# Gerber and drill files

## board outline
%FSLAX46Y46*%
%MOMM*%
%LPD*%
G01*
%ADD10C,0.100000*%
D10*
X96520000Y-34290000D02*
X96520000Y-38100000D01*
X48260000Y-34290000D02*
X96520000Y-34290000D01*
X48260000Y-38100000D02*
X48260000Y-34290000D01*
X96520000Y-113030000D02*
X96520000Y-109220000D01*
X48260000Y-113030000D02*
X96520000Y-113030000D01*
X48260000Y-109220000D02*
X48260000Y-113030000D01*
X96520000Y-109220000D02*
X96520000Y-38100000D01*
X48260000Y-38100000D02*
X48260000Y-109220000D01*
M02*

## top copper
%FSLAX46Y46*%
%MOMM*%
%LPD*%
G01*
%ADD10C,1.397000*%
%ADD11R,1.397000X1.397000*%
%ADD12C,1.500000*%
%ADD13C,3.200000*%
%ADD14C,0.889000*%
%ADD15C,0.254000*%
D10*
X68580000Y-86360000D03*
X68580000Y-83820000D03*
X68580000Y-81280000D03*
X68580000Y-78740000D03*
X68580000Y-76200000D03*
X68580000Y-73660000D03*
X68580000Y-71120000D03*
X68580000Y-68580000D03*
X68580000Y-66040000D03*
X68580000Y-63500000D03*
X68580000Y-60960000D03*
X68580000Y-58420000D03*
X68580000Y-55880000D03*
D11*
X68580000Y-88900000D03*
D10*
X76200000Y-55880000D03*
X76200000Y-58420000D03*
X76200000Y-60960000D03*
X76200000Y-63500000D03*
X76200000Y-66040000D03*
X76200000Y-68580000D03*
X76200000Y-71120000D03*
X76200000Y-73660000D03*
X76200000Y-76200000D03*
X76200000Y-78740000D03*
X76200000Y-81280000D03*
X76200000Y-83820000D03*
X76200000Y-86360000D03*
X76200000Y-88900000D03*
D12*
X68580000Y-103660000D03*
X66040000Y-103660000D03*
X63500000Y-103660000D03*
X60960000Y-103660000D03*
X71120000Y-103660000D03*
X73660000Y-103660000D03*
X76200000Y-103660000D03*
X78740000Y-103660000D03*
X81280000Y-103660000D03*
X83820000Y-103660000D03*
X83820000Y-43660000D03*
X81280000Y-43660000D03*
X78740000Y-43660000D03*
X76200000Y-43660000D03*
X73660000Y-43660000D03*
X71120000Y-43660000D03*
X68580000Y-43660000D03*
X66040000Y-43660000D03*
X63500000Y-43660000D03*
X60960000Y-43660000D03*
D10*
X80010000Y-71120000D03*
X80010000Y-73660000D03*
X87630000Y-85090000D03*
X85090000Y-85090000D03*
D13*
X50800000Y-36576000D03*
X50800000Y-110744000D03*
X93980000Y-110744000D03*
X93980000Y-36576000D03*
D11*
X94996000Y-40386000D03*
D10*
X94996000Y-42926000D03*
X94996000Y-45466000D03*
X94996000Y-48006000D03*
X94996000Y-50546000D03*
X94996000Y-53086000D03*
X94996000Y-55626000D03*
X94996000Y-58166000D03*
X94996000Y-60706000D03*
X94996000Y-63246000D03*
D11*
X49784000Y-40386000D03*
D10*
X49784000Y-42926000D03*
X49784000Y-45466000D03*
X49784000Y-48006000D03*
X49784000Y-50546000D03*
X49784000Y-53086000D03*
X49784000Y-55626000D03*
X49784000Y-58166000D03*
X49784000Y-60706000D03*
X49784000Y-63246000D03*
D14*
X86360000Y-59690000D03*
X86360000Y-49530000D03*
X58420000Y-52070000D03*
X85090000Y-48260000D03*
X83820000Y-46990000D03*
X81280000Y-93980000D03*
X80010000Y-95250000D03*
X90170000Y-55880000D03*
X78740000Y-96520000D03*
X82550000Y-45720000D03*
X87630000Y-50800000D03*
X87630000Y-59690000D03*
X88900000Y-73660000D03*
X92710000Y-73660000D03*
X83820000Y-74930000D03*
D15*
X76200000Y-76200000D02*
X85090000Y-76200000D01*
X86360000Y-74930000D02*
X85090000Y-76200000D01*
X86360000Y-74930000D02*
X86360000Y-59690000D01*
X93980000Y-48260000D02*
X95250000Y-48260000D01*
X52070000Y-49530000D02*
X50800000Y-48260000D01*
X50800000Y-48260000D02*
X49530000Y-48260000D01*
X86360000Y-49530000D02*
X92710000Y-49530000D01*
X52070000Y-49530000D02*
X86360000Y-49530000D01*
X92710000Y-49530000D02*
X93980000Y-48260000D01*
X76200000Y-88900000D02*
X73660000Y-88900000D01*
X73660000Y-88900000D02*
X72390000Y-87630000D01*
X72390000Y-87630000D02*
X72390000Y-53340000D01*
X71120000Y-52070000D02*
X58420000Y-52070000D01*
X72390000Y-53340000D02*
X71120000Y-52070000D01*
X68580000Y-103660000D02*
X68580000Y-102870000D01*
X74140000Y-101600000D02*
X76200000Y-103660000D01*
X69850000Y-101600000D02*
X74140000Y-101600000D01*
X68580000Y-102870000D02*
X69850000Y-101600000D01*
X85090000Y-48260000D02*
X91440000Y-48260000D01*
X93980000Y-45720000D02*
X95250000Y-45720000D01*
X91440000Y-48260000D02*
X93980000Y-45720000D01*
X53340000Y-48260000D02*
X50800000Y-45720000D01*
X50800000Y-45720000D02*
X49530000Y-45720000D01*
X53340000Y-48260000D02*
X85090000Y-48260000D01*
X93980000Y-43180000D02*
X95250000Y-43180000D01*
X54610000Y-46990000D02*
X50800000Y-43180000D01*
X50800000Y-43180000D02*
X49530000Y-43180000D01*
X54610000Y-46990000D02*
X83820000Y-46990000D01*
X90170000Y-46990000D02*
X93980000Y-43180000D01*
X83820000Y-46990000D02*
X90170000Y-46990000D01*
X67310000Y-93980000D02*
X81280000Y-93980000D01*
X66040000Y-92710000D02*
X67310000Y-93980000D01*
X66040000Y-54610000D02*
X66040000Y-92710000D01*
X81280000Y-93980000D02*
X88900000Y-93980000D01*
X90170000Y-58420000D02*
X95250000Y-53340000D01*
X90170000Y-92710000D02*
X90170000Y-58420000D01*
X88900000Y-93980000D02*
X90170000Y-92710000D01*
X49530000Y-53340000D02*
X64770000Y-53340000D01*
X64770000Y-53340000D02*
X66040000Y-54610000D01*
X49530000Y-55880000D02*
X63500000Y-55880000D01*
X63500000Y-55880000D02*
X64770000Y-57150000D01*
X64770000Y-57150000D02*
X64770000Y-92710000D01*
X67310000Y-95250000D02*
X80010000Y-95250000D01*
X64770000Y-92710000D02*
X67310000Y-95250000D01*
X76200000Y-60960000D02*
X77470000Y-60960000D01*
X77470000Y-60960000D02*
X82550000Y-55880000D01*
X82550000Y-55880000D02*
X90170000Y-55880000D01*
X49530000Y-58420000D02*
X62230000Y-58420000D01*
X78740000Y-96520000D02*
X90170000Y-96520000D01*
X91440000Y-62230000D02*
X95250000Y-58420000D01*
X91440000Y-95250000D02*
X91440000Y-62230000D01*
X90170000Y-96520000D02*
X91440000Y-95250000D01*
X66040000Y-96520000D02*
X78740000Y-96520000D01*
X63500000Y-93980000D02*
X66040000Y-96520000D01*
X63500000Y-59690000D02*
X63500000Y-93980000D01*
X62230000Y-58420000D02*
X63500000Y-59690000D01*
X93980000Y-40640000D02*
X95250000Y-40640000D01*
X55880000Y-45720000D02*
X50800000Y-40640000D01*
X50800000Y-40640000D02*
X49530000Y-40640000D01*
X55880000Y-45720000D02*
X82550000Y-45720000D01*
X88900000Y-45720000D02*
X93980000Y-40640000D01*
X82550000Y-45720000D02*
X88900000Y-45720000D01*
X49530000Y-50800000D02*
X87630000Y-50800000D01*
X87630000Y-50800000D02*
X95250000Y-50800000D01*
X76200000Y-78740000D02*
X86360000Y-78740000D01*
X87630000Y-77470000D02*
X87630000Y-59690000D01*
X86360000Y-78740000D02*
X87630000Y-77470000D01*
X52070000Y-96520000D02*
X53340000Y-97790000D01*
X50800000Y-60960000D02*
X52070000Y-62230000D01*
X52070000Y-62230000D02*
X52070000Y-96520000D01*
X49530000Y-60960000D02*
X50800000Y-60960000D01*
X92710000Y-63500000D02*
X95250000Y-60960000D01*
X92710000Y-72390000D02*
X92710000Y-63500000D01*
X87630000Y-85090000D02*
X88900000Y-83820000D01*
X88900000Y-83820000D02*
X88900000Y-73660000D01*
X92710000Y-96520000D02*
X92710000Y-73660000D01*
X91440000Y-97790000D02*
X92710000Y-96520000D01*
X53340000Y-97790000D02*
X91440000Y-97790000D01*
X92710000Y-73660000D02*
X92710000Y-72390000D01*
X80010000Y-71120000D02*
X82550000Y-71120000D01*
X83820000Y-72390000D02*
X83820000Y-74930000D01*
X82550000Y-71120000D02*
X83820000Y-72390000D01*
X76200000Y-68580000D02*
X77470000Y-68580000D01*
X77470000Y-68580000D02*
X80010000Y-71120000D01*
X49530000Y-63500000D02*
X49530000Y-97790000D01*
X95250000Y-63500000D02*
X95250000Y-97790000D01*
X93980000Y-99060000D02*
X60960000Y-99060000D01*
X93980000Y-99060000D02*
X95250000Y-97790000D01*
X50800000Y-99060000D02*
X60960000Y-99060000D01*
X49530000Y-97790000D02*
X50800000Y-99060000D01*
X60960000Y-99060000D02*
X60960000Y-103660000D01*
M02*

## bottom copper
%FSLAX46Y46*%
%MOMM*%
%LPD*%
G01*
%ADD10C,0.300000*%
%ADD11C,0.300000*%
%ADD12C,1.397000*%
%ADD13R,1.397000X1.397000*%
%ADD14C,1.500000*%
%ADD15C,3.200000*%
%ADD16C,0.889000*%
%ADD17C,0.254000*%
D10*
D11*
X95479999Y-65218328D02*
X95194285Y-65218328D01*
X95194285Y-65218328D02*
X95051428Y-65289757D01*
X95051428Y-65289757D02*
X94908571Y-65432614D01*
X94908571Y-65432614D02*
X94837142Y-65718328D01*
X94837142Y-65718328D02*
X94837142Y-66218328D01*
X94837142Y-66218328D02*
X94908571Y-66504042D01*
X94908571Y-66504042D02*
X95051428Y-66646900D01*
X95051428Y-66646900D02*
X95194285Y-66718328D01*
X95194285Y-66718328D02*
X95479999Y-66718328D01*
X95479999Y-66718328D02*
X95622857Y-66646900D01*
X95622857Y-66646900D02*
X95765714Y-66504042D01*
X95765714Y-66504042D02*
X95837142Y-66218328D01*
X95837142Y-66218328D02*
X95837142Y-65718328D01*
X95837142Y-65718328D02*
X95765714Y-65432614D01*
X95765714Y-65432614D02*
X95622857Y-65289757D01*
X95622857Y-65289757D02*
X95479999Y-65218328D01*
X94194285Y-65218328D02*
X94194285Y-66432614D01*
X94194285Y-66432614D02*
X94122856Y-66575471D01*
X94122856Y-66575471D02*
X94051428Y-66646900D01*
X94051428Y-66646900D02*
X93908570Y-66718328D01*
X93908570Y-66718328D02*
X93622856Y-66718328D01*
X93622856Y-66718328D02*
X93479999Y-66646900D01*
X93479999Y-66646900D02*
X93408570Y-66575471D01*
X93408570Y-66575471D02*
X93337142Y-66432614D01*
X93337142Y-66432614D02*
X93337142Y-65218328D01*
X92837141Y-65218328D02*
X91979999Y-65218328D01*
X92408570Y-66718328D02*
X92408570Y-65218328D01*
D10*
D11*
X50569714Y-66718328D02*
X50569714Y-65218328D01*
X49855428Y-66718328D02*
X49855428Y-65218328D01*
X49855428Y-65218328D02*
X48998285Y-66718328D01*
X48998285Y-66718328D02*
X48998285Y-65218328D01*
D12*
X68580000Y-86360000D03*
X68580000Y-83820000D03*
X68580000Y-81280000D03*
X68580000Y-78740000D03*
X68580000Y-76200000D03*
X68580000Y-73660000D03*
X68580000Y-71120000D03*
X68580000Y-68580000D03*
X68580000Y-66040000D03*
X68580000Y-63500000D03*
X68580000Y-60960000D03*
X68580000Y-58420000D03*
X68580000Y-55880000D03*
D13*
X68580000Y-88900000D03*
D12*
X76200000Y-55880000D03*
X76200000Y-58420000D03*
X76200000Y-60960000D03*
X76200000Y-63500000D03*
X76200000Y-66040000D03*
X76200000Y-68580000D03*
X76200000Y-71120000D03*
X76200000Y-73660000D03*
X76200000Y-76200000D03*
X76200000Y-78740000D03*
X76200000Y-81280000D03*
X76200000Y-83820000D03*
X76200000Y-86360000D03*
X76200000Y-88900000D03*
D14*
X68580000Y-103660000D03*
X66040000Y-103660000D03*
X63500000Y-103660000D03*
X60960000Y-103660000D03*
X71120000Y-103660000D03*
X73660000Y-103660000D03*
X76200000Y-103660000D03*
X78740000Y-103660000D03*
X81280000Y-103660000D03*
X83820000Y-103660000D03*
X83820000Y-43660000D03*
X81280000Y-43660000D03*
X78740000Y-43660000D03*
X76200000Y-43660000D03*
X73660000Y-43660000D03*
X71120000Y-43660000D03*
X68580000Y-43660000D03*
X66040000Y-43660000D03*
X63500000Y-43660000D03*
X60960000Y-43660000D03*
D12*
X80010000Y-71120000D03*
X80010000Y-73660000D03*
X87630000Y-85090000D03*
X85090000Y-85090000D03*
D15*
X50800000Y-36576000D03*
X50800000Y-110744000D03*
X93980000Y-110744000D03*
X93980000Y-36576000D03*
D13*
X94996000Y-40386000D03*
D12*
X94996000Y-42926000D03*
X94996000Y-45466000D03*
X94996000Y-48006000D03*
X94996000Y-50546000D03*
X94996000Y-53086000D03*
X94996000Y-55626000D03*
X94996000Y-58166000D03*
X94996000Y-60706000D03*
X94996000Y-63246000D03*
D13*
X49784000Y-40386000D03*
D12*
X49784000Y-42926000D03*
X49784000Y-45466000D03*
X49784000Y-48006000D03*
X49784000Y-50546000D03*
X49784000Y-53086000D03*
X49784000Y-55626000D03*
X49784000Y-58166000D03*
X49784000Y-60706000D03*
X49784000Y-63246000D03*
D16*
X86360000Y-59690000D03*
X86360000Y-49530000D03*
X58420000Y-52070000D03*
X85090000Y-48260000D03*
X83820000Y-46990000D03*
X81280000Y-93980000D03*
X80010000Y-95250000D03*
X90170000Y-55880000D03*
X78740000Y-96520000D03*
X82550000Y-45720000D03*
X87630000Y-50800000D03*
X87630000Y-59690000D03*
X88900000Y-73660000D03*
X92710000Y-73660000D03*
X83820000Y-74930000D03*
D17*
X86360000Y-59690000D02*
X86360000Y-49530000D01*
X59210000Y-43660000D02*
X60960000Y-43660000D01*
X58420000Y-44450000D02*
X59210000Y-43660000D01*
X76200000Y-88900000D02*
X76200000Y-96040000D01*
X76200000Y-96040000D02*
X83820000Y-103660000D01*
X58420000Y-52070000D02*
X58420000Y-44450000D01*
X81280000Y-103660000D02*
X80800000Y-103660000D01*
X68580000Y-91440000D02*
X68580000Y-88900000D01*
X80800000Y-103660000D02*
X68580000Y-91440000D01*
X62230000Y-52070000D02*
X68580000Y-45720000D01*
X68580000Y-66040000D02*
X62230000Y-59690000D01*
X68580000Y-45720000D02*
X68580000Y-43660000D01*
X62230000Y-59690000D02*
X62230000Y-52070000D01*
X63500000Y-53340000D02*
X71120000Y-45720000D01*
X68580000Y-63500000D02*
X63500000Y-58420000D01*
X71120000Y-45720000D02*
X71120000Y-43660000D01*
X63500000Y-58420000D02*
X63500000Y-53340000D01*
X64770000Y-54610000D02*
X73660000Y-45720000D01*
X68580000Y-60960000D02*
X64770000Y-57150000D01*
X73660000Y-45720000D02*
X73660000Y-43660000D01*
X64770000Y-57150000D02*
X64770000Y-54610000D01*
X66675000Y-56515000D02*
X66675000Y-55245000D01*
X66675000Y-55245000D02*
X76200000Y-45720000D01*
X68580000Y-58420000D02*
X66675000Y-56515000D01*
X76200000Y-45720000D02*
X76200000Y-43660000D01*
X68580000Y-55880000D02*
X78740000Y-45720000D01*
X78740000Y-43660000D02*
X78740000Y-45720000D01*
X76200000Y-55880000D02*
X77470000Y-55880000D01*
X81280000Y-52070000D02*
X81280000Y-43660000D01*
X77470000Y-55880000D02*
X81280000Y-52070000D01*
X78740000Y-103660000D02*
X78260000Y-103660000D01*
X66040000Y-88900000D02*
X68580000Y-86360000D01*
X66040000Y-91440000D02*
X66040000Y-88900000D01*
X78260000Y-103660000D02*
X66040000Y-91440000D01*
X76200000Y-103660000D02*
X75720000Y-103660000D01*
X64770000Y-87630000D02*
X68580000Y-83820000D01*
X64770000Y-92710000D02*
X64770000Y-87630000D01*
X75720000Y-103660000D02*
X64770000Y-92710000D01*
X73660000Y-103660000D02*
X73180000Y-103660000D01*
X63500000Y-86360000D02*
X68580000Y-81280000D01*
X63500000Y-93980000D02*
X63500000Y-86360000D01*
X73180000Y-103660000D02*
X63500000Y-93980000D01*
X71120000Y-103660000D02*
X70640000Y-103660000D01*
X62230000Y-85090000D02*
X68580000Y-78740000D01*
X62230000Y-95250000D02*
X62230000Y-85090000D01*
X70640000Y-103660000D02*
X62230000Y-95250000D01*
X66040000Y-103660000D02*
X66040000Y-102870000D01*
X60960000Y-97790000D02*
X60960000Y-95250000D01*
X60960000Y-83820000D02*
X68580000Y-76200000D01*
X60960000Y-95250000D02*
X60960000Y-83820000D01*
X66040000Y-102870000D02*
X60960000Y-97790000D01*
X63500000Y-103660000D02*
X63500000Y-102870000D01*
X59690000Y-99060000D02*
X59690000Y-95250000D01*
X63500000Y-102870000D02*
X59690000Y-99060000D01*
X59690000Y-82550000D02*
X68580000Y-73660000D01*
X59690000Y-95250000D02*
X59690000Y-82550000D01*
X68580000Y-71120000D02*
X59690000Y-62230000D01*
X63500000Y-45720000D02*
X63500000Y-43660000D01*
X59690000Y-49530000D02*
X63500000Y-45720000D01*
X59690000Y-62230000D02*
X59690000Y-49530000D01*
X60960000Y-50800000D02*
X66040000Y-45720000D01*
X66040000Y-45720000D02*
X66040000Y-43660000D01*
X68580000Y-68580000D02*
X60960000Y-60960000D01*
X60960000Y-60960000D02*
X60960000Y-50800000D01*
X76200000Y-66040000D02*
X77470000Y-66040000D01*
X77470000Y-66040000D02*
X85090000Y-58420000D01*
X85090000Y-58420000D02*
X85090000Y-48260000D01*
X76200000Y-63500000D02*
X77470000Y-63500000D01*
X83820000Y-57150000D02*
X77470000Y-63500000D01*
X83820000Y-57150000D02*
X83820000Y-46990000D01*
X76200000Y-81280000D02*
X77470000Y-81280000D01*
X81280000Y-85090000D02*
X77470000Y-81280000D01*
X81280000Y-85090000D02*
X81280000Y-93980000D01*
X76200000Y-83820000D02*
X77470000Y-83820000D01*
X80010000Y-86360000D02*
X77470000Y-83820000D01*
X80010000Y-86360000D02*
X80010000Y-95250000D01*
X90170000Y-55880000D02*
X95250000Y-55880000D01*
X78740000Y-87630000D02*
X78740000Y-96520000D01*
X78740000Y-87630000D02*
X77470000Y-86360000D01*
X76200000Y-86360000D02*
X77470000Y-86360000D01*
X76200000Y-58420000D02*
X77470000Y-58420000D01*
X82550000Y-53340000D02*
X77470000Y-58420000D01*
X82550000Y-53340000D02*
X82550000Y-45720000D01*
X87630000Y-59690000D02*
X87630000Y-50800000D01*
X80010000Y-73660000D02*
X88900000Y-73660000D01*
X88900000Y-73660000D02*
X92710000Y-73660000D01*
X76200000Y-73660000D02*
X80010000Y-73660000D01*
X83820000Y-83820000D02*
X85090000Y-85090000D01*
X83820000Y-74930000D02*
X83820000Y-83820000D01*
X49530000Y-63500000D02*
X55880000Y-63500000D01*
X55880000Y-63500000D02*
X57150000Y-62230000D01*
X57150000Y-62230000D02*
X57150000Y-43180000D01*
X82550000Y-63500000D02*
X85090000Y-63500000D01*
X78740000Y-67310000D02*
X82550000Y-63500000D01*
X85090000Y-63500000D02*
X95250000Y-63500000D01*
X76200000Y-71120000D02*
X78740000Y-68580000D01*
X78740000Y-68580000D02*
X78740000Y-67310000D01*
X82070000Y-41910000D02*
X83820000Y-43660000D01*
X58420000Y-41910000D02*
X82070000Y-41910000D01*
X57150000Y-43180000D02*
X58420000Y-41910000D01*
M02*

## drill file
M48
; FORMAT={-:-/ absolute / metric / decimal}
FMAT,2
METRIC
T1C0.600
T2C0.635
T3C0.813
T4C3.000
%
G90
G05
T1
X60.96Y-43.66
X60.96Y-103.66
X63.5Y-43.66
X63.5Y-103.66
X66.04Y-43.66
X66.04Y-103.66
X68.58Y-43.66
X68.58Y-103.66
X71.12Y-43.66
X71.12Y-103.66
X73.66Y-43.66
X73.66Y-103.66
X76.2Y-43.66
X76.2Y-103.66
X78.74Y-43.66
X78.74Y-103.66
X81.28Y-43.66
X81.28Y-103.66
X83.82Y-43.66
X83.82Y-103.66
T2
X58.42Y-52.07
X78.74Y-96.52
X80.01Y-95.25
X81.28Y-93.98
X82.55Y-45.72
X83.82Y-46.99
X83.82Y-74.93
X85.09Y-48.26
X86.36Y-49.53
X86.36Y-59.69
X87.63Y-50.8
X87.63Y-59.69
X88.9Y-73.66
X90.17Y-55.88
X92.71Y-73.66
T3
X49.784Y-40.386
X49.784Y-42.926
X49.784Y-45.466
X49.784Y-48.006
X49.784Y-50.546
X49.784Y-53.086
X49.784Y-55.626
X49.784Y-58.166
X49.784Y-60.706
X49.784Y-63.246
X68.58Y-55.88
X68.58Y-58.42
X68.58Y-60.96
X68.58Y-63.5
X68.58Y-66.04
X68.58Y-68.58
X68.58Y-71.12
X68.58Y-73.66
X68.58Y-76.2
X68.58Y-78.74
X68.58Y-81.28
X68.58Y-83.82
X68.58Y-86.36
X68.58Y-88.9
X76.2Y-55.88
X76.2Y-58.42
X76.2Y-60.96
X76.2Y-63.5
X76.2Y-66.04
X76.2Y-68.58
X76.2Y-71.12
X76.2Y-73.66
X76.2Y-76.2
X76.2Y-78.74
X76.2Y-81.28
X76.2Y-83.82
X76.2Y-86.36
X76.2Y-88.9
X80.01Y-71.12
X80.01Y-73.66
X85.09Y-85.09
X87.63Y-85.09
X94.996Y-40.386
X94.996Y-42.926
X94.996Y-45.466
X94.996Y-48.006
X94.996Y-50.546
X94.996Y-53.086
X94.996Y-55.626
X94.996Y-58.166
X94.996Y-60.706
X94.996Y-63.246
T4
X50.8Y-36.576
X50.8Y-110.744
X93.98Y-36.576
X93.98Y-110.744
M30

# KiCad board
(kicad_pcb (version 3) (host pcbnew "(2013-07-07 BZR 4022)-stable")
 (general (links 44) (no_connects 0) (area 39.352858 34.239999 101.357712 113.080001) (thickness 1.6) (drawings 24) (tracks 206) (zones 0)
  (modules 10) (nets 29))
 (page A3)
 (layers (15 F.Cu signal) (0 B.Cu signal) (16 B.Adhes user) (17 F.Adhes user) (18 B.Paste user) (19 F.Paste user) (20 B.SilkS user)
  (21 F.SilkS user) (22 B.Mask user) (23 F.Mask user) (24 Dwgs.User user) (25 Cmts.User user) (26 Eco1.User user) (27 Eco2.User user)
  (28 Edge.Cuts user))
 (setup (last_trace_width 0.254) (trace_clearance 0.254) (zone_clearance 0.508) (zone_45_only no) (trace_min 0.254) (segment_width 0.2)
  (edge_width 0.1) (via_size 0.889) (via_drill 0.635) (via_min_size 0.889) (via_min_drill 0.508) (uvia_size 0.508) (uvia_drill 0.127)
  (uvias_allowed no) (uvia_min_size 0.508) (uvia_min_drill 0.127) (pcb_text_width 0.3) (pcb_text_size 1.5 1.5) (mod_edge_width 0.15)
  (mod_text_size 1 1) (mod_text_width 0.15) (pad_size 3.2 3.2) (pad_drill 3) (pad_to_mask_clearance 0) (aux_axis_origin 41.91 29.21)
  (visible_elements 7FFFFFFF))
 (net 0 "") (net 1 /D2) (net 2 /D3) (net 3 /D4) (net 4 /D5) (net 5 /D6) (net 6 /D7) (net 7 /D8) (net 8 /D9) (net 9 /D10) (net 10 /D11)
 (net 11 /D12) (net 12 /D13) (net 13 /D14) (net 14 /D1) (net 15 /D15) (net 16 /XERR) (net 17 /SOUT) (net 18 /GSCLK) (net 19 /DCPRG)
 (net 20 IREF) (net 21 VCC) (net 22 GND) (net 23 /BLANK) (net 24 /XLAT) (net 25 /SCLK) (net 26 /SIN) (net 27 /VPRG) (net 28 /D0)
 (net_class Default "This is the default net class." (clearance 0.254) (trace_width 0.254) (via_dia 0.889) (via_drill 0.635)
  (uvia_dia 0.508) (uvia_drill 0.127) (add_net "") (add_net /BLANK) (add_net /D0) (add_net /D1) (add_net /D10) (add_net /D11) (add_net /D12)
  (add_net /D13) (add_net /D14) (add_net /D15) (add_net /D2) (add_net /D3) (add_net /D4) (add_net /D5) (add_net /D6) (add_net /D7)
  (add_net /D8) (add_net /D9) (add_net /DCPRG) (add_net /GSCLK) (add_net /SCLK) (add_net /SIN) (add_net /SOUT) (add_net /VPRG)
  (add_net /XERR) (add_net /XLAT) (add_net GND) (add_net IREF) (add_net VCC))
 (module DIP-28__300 (layer B.Cu) (at 72.39 72.39 90)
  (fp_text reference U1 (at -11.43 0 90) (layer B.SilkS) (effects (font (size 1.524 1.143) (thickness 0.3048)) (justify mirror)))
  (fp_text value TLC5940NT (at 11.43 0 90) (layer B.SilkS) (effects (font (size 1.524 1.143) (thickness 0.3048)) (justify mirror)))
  (pad 2 thru_hole circle (at -13.97 -3.81 90) (size 1.397 1.397) (drill 0.8128) (layers *.Cu *.Mask B.SilkS) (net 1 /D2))
  (pad 3 thru_hole circle (at -11.43 -3.81 90) (size 1.397 1.397) (drill 0.8128) (layers *.Cu *.Mask B.SilkS) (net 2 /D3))
  (pad 4 thru_hole circle (at -8.89 -3.81 90) (size 1.397 1.397) (drill 0.8128) (layers *.Cu *.Mask B.SilkS) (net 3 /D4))
  (pad 5 thru_hole circle (at -6.35 -3.81 90) (size 1.397 1.397) (drill 0.8128) (layers *.Cu *.Mask B.SilkS) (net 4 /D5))
  (pad 6 thru_hole circle (at -3.81 -3.81 90) (size 1.397 1.397) (drill 0.8128) (layers *.Cu *.Mask B.SilkS) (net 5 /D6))
  (pad 7 thru_hole circle (at -1.27 -3.81 90) (size 1.397 1.397) (drill 0.8128) (layers *.Cu *.Mask B.SilkS) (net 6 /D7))
  (pad 8 thru_hole circle (at 1.27 -3.81 90) (size 1.397 1.397) (drill 0.8128) (layers *.Cu *.Mask B.SilkS) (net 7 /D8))
  (pad 9 thru_hole circle (at 3.81 -3.81 90) (size 1.397 1.397) (drill 0.8128) (layers *.Cu *.Mask B.SilkS) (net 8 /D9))
  (pad 10 thru_hole circle (at 6.35 -3.81 90) (size 1.397 1.397) (drill 0.8128) (layers *.Cu *.Mask B.SilkS) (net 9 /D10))
  (pad 11 thru_hole circle (at 8.89 -3.81 90) (size 1.397 1.397) (drill 0.8128) (layers *.Cu *.Mask B.SilkS) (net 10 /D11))
  (pad 12 thru_hole circle (at 11.43 -3.81 90) (size 1.397 1.397) (drill 0.8128) (layers *.Cu *.Mask B.SilkS) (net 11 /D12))
  (pad 13 thru_hole circle (at 13.97 -3.81 90) (size 1.397 1.397) (drill 0.8128) (layers *.Cu *.Mask B.SilkS) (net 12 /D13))
  (pad 14 thru_hole circle (at 16.51 -3.81 90) (size 1.397 1.397) (drill 0.8128) (layers *.Cu *.Mask B.SilkS) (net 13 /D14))
  (pad 1 thru_hole rect (at -16.51 -3.81 90) (size 1.397 1.397) (drill 0.8128) (layers *.Cu *.Mask B.SilkS) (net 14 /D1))
  (pad 15 thru_hole circle (at 16.51 3.81 90) (size 1.397 1.397) (drill 0.8128) (layers *.Cu *.Mask B.SilkS) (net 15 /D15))
  (pad 16 thru_hole circle (at 13.97 3.81 90) (size 1.397 1.397) (drill 0.8128) (layers *.Cu *.Mask B.SilkS) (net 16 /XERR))
  (pad 17 thru_hole circle (at 11.43 3.81 90) (size 1.397 1.397) (drill 0.8128) (layers *.Cu *.Mask B.SilkS) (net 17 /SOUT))
  (pad 18 thru_hole circle (at 8.89 3.81 90) (size 1.397 1.397) (drill 0.8128) (layers *.Cu *.Mask B.SilkS) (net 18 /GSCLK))
  (pad 19 thru_hole circle (at 6.35 3.81 90) (size 1.397 1.397) (drill 0.8128) (layers *.Cu *.Mask B.SilkS) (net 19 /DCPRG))
  (pad 20 thru_hole circle (at 3.81 3.81 90) (size 1.397 1.397) (drill 0.8128) (layers *.Cu *.Mask B.SilkS) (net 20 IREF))
  (pad 21 thru_hole circle (at 1.27 3.81 90) (size 1.397 1.397) (drill 0.8128) (layers *.Cu *.Mask B.SilkS) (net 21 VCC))
  (pad 22 thru_hole circle (at -1.27 3.81 90) (size 1.397 1.397) (drill 0.8128) (layers *.Cu *.Mask B.SilkS) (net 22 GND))
  (pad 23 thru_hole circle (at -3.81 3.81 90) (size 1.397 1.397) (drill 0.8128) (layers *.Cu *.Mask B.SilkS) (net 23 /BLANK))
  (pad 24 thru_hole circle (at -6.35 3.81 90) (size 1.397 1.397) (drill 0.8128) (layers *.Cu *.Mask B.SilkS) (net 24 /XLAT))
  (pad 25 thru_hole circle (at -8.89 3.81 90) (size 1.397 1.397) (drill 0.8128) (layers *.Cu *.Mask B.SilkS) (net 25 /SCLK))
  (pad 26 thru_hole circle (at -11.43 3.81 90) (size 1.397 1.397) (drill 0.8128) (layers *.Cu *.Mask B.SilkS) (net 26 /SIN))
  (pad 27 thru_hole circle (at -13.97 3.81 90) (size 1.397 1.397) (drill 0.8128) (layers *.Cu *.Mask B.SilkS) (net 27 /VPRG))
  (pad 28 thru_hole circle (at -16.51 3.81 90) (size 1.397 1.397) (drill 0.8128) (layers *.Cu *.Mask B.SilkS) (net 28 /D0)))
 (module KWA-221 (layer F.Cu) (at 72.39 73.66)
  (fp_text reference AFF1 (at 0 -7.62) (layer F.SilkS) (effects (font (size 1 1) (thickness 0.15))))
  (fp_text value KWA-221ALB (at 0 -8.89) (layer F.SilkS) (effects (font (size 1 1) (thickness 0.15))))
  (pad 4 thru_hole circle (at -3.81 30) (size 1.5 1.5) (drill 0.6) (layers *.Cu *.Mask F.SilkS) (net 2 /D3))
  (pad 3 thru_hole circle (at -6.35 30) (size 1.5 1.5) (drill 0.6) (layers *.Cu *.Mask F.SilkS) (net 5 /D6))
  (pad 2 thru_hole circle (at -8.89 30) (size 1.5 1.5) (drill 0.6) (layers *.Cu *.Mask F.SilkS) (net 6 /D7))
  (pad 1 thru_hole circle (at -11.43 30) (size 1.5 1.5) (drill 0.6) (layers *.Cu *.Mask F.SilkS) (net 21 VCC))
  (pad 5 thru_hole circle (at -1.27 30) (size 1.5 1.5) (drill 0.6) (layers *.Cu *.Mask F.SilkS) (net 4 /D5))
  (pad 6 thru_hole circle (at 1.27 30) (size 1.5 1.5) (drill 0.6) (layers *.Cu *.Mask F.SilkS) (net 3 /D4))
  (pad 7 thru_hole circle (at 3.81 30) (size 1.5 1.5) (drill 0.6) (layers *.Cu *.Mask F.SilkS) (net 2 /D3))
  (pad 8 thru_hole circle (at 6.35 30) (size 1.5 1.5) (drill 0.6) (layers *.Cu *.Mask F.SilkS) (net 1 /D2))
  (pad 9 thru_hole circle (at 8.89 30) (size 1.5 1.5) (drill 0.6) (layers *.Cu *.Mask F.SilkS) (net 14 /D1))
  (pad 10 thru_hole circle (at 11.43 30) (size 1.5 1.5) (drill 0.6) (layers *.Cu *.Mask F.SilkS) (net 28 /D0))
  (pad 11 thru_hole circle (at 11.43 -30) (size 1.5 1.5) (drill 0.6) (layers *.Cu *.Mask F.SilkS) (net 21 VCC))
  (pad 12 thru_hole circle (at 8.89 -30) (size 1.5 1.5) (drill 0.6) (layers *.Cu *.Mask F.SilkS) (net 15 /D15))
  (pad 13 thru_hole circle (at 6.35 -30) (size 1.5 1.5) (drill 0.6) (layers *.Cu *.Mask F.SilkS) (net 13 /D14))
  (pad 14 thru_hole circle (at 3.81 -30) (size 1.5 1.5) (drill 0.6) (layers *.Cu *.Mask F.SilkS) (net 12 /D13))
  (pad 15 thru_hole circle (at 1.27 -30) (size 1.5 1.5) (drill 0.6) (layers *.Cu *.Mask F.SilkS) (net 11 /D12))
  (pad 16 thru_hole circle (at -1.27 -30) (size 1.5 1.5) (drill 0.6) (layers *.Cu *.Mask F.SilkS) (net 10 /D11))
  (pad 17 thru_hole circle (at -3.81 -30) (size 1.5 1.5) (drill 0.6) (layers *.Cu *.Mask F.SilkS) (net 9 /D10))
  (pad 18 thru_hole circle (at -6.35 -30) (size 1.5 1.5) (drill 0.6) (layers *.Cu *.Mask F.SilkS) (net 8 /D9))
  (pad 19 thru_hole circle (at -8.89 -30) (size 1.5 1.5) (drill 0.6) (layers *.Cu *.Mask F.SilkS) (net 7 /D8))
  (pad 20 thru_hole circle (at -11.43 -30) (size 1.5 1.5) (drill 0.6) (layers *.Cu *.Mask F.SilkS) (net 28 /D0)))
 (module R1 (layer B.Cu) (at 80.01 72.39 270) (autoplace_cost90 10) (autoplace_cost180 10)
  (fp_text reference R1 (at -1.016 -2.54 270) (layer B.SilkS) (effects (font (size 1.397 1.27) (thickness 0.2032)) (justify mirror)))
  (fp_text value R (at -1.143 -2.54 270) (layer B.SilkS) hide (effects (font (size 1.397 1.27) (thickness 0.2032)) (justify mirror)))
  (pad 1 thru_hole circle (at -1.27 0 270) (size 1.397 1.397) (drill 0.8128) (layers *.Cu *.Mask B.SilkS) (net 20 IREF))
  (pad 2 thru_hole circle (at 1.27 0 270) (size 1.397 1.397) (drill 0.8128) (layers *.Cu *.Mask B.SilkS) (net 22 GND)))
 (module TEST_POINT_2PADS (layer F.Cu) (at 86.36 85.09 180)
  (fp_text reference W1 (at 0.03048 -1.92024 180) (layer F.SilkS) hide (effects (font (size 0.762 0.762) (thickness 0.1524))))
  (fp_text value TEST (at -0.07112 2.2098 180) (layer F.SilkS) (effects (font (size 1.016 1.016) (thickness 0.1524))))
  (pad 1 thru_hole circle (at -1.27 0 180) (size 1.397 1.397) (drill 0.8128) (layers *.Cu *.Mask F.SilkS) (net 22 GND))
  (pad 2 thru_hole circle (at 1.27 0 180) (size 1.397 1.397) (drill 0.8128) (layers *.Cu *.Mask F.SilkS) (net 20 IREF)))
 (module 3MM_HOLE (layer F.Cu) (at 50.8 36.576)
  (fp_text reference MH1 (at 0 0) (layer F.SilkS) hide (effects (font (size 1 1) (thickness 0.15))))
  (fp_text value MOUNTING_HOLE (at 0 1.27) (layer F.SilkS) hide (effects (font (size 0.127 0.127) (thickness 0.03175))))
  (pad "" thru_hole circle (at 0 0) (size 3.2 3.2) (drill 3) (layers *.Cu *.Mask)))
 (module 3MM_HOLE (layer F.Cu) (at 50.8 110.744)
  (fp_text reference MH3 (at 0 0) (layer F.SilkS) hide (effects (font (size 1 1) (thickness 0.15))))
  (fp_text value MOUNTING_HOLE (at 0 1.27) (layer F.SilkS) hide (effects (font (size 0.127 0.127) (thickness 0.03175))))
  (pad "" thru_hole circle (at 0 0) (size 3.2 3.2) (drill 3) (layers *.Cu *.Mask)))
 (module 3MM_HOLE (layer F.Cu) (at 93.98 110.744)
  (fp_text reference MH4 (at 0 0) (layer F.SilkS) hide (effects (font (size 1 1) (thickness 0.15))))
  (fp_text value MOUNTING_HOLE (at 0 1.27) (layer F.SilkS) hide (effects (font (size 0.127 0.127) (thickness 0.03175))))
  (pad "" thru_hole circle (at 0 0) (size 3.2 3.2) (drill 3) (layers *.Cu *.Mask)))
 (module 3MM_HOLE (layer F.Cu) (at 93.98 36.576)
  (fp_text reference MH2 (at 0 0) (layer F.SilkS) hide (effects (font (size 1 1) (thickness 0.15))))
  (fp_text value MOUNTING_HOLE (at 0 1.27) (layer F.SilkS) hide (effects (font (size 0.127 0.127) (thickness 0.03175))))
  (pad "" thru_hole circle (at 0 0) (size 3.2 3.2) (drill 3) (layers *.Cu *.Mask)))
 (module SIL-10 (layer B.Cu) (at 94.996 51.816 270)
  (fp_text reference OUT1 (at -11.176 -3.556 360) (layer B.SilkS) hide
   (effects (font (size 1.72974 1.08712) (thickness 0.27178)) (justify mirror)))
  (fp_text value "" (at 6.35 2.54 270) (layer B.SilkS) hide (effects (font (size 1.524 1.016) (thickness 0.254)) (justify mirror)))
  (pad 1 thru_hole rect (at -11.43 0 270) (size 1.397 1.397) (drill 0.8128) (layers *.Cu *.Mask B.SilkS) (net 16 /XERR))
  (pad 2 thru_hole circle (at -8.89 0 270) (size 1.397 1.397) (drill 0.8128) (layers *.Cu *.Mask B.SilkS) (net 18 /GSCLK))
  (pad 3 thru_hole circle (at -6.35 0 270) (size 1.397 1.397) (drill 0.8128) (layers *.Cu *.Mask B.SilkS) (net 19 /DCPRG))
  (pad 4 thru_hole circle (at -3.81 0 270) (size 1.397 1.397) (drill 0.8128) (layers *.Cu *.Mask B.SilkS) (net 23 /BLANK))
  (pad 5 thru_hole circle (at -1.27 0 270) (size 1.397 1.397) (drill 0.8128) (layers *.Cu *.Mask B.SilkS) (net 24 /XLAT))
  (pad 6 thru_hole circle (at 1.27 0 270) (size 1.397 1.397) (drill 0.8128) (layers *.Cu *.Mask B.SilkS) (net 25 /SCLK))
  (pad 7 thru_hole circle (at 3.81 0 270) (size 1.397 1.397) (drill 0.8128) (layers *.Cu *.Mask B.SilkS) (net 17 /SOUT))
  (pad 8 thru_hole circle (at 6.35 0 270) (size 1.397 1.397) (drill 0.8128) (layers *.Cu *.Mask B.SilkS) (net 27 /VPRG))
  (pad 9 thru_hole circle (at 8.89 0 270) (size 1.397 1.397) (drill 0.8128) (layers *.Cu *.Mask B.SilkS) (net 22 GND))
  (pad 10 thru_hole circle (at 11.43 0 270) (size 1.397 1.397) (drill 0.8128) (layers *.Cu *.Mask B.SilkS) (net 21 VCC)))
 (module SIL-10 (layer B.Cu) (at 49.784 51.816 270)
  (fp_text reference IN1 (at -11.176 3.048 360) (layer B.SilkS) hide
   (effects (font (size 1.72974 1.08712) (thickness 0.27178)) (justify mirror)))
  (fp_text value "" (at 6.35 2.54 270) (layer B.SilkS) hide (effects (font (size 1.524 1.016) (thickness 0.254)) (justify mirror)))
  (pad 1 thru_hole rect (at -11.43 0 270) (size 1.397 1.397) (drill 0.8128) (layers *.Cu *.Mask B.SilkS) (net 16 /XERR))
  (pad 2 thru_hole circle (at -8.89 0 270) (size 1.397 1.397) (drill 0.8128) (layers *.Cu *.Mask B.SilkS) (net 18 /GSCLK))
  (pad 3 thru_hole circle (at -6.35 0 270) (size 1.397 1.397) (drill 0.8128) (layers *.Cu *.Mask B.SilkS) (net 19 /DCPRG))
  (pad 4 thru_hole circle (at -3.81 0 270) (size 1.397 1.397) (drill 0.8128) (layers *.Cu *.Mask B.SilkS) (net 23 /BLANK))
  (pad 5 thru_hole circle (at -1.27 0 270) (size 1.397 1.397) (drill 0.8128) (layers *.Cu *.Mask B.SilkS) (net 24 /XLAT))
  (pad 6 thru_hole circle (at 1.27 0 270) (size 1.397 1.397) (drill 0.8128) (layers *.Cu *.Mask B.SilkS) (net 25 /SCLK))
  (pad 7 thru_hole circle (at 3.81 0 270) (size 1.397 1.397) (drill 0.8128) (layers *.Cu *.Mask B.SilkS) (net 26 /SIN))
  (pad 8 thru_hole circle (at 6.35 0 270) (size 1.397 1.397) (drill 0.8128) (layers *.Cu *.Mask B.SilkS) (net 27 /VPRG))
  (pad 9 thru_hole circle (at 8.89 0 270) (size 1.397 1.397) (drill 0.8128) (layers *.Cu *.Mask B.SilkS) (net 22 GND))
  (pad 10 thru_hole circle (at 11.43 0 270) (size 1.397 1.397) (drill 0.8128) (layers *.Cu *.Mask B.SilkS) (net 21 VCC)))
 (gr_line (start 96.52 34.29) (end 96.52 38.1) (angle 90) (layer Edge.Cuts) (width 0.1))
 (gr_line (start 48.26 34.29) (end 96.52 34.29) (angle 90) (layer Edge.Cuts) (width 0.1))
 (gr_line (start 48.26 38.1) (end 48.26 34.29) (angle 90) (layer Edge.Cuts) (width 0.1))
 (gr_line (start 96.52 113.03) (end 96.52 109.22) (angle 90) (layer Edge.Cuts) (width 0.1))
 (gr_line (start 48.26 113.03) (end 96.52 113.03) (angle 90) (layer Edge.Cuts) (width 0.1))
 (gr_line (start 48.26 109.22) (end 48.26 113.03) (angle 90) (layer Edge.Cuts) (width 0.1))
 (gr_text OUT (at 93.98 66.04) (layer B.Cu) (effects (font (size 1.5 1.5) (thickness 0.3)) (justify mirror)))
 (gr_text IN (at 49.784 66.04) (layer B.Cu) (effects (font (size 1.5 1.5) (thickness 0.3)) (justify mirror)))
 (gr_line (start 96.52 109.22) (end 96.52 38.1) (angle 90) (layer Edge.Cuts) (width 0.1))
 (gr_line (start 48.26 38.1) (end 48.26 109.22) (angle 90) (layer Edge.Cuts) (width 0.1))
 (via (at 86.36 59.69) (size 0.889) (layers F.Cu B.Cu) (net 23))
 (segment (start 76.2 76.2) (end 85.09 76.2) (width 0.254) (layer F.Cu) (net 23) (status 10))
 (segment (start 86.36 74.93) (end 85.09 76.2) (width 0.254) (layer F.Cu) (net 23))
 (segment (start 86.36 74.93) (end 86.36 59.69) (width 0.254) (layer F.Cu) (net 23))
 (segment (start 93.98 48.26) (end 95.25 48.26) (width 0.254) (layer F.Cu) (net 23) (status 20))
 (segment (start 52.07 49.53) (end 50.8 48.26) (width 0.254) (layer F.Cu) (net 23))
 (segment (start 50.8 48.26) (end 49.53 48.26) (width 0.254) (layer F.Cu) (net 23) (status 20))
 (via (at 86.36 49.53) (size 0.889) (layers F.Cu B.Cu) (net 23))
 (segment (start 86.36 59.69) (end 86.36 49.53) (width 0.254) (layer B.Cu) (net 23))
 (segment (start 86.36 49.53) (end 92.71 49.53) (width 0.254) (layer F.Cu) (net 23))
 (segment (start 52.07 49.53) (end 86.36 49.53) (width 0.254) (layer F.Cu) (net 23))
 (segment (start 92.71 49.53) (end 93.98 48.26) (width 0.254) (layer F.Cu) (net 23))
 (segment (start 76.2 88.9) (end 73.66 88.9) (width 0.254) (layer F.Cu) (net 28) (status 10))
 (segment (start 59.21 43.66) (end 60.96 43.66) (width 0.254) (layer B.Cu) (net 28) (status 20))
 (segment (start 58.42 44.45) (end 59.21 43.66) (width 0.254) (layer B.Cu) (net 28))
 (segment (start 73.66 88.9) (end 72.39 87.63) (width 0.254) (layer F.Cu) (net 28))
 (segment (start 76.2 88.9) (end 76.2 96.04) (width 0.254) (layer B.Cu) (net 28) (status 10))
 (segment (start 76.2 96.04) (end 83.82 103.66) (width 0.254) (layer B.Cu) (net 28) (status 20))
 (segment (start 72.39 87.63) (end 72.39 53.34) (width 0.254) (layer F.Cu) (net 28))
 (segment (start 58.42 52.07) (end 58.42 44.45) (width 0.254) (layer B.Cu) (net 28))
 (via (at 58.42 52.07) (size 0.889) (layers F.Cu B.Cu) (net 28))
 (segment (start 71.12 52.07) (end 58.42 52.07) (width 0.254) (layer F.Cu) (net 28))
 (segment (start 72.39 53.34) (end 71.12 52.07) (width 0.254) (layer F.Cu) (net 28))
 (segment (start 81.28 103.66) (end 80.8 103.66) (width 0.254) (layer B.Cu) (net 14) (status 30))
 (segment (start 68.58 91.44) (end 68.58 88.9) (width 0.254) (layer B.Cu) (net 14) (status 20))
 (segment (start 80.8 103.66) (end 68.58 91.44) (width 0.254) (layer B.Cu) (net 14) (status 10))
 (segment (start 62.23 52.07) (end 68.58 45.72) (width 0.254) (layer B.Cu) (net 9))
 (segment (start 68.58 66.04) (end 62.23 59.69) (width 0.254) (layer B.Cu) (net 9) (status 10))
 (segment (start 68.58 45.72) (end 68.58 43.66) (width 0.254) (layer B.Cu) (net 9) (status 20))
 (segment (start 62.23 59.69) (end 62.23 52.07) (width 0.254) (layer B.Cu) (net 9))
 (segment (start 63.5 53.34) (end 71.12 45.72) (width 0.254) (layer B.Cu) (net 10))
 (segment (start 68.58 63.5) (end 63.5 58.42) (width 0.254) (layer B.Cu) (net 10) (status 10))
 (segment (start 71.12 45.72) (end 71.12 43.66) (width 0.254) (layer B.Cu) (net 10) (status 20))
 (segment (start 63.5 58.42) (end 63.5 53.34) (width 0.254) (layer B.Cu) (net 10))
 (segment (start 64.77 54.61) (end 73.66 45.72) (width 0.254) (layer B.Cu) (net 11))
 (segment (start 68.58 60.96) (end 64.77 57.15) (width 0.254) (layer B.Cu) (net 11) (status 10))
 (segment (start 73.66 45.72) (end 73.66 43.66) (width 0.254) (layer B.Cu) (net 11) (status 20))
 (segment (start 64.77 57.15) (end 64.77 54.61) (width 0.254) (layer B.Cu) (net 11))
 (segment (start 66.675 56.515) (end 66.675 55.245) (width 0.254) (layer B.Cu) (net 12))
 (segment (start 66.675 55.245) (end 76.2 45.72) (width 0.254) (layer B.Cu) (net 12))
 (segment (start 68.58 58.42) (end 66.675 56.515) (width 0.254) (layer B.Cu) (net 12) (status 10))
 (segment (start 76.2 45.72) (end 76.2 43.66) (width 0.254) (layer B.Cu) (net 12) (status 20))
 (segment (start 68.58 55.88) (end 78.74 45.72) (width 0.254) (layer B.Cu) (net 13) (status 10))
 (segment (start 78.74 43.66) (end 78.74 45.72) (width 0.254) (layer B.Cu) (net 13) (status 10))
 (segment (start 76.2 55.88) (end 77.47 55.88) (width 0.254) (layer B.Cu) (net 15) (status 10))
 (segment (start 81.28 52.07) (end 81.28 43.66) (width 0.254) (layer B.Cu) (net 15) (status 20))
 (segment (start 77.47 55.88) (end 81.28 52.07) (width 0.254) (layer B.Cu) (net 15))
 (segment (start 78.74 103.66) (end 78.26 103.66) (width 0.254) (layer B.Cu) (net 1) (status 30))
 (segment (start 66.04 88.9) (end 68.58 86.36) (width 0.254) (layer B.Cu) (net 1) (status 20))
 (segment (start 66.04 91.44) (end 66.04 88.9) (width 0.254) (layer B.Cu) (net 1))
 (segment (start 78.26 103.66) (end 66.04 91.44) (width 0.254) (layer B.Cu) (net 1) (status 10))
 (segment (start 68.58 103.66) (end 68.58 102.87) (width 0.254) (layer F.Cu) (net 2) (status 10))
 (segment (start 74.14 101.6) (end 76.2 103.66) (width 0.254) (layer F.Cu) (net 2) (status 20))
 (segment (start 69.85 101.6) (end 74.14 101.6) (width 0.254) (layer F.Cu) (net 2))
 (segment (start 68.58 102.87) (end 69.85 101.6) (width 0.254) (layer F.Cu) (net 2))
 (segment (start 76.2 103.66) (end 75.72 103.66) (width 0.254) (layer B.Cu) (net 2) (status 30))
 (segment (start 64.77 87.63) (end 68.58 83.82) (width 0.254) (layer B.Cu) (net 2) (status 20))
 (segment (start 64.77 92.71) (end 64.77 87.63) (width 0.254) (layer B.Cu) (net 2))
 (segment (start 75.72 103.66) (end 64.77 92.71) (width 0.254) (layer B.Cu) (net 2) (status 10))
 (segment (start 73.66 103.66) (end 73.18 103.66) (width 0.254) (layer B.Cu) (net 3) (status 30))
 (segment (start 63.5 86.36) (end 68.58 81.28) (width 0.254) (layer B.Cu) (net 3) (status 20))
 (segment (start 63.5 93.98) (end 63.5 86.36) (width 0.254) (layer B.Cu) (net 3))
 (segment (start 73.18 103.66) (end 63.5 93.98) (width 0.254) (layer B.Cu) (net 3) (status 10))
 (segment (start 71.12 103.66) (end 70.64 103.66) (width 0.254) (layer B.Cu) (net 4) (status 30))
 (segment (start 62.23 85.09) (end 68.58 78.74) (width 0.254) (layer B.Cu) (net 4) (status 20))
 (segment (start 62.23 95.25) (end 62.23 85.09) (width 0.254) (layer B.Cu) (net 4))
 (segment (start 70.64 103.66) (end 62.23 95.25) (width 0.254) (layer B.Cu) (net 4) (status 10))
 (segment (start 66.04 103.66) (end 66.04 102.87) (width 0.254) (layer B.Cu) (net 5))
 (segment (start 60.96 97.79) (end 60.96 95.25) (width 0.254) (layer B.Cu) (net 5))
 (segment (start 60.96 83.82) (end 68.58 76.2) (width 0.254) (layer B.Cu) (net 5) (status 20))
 (segment (start 60.96 95.25) (end 60.96 83.82) (width 0.254) (layer B.Cu) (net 5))
 (segment (start 66.04 102.87) (end 60.96 97.79) (width 0.254) (layer B.Cu) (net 5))
 (segment (start 63.5 103.66) (end 63.5 102.87) (width 0.254) (layer B.Cu) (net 6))
 (segment (start 59.69 99.06) (end 59.69 95.25) (width 0.254) (layer B.Cu) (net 6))
 (segment (start 63.5 102.87) (end 59.69 99.06) (width 0.254) (layer B.Cu) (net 6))
 (segment (start 59.69 82.55) (end 68.58 73.66) (width 0.254) (layer B.Cu) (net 6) (status 20))
 (segment (start 59.69 95.25) (end 59.69 82.55) (width 0.254) (layer B.Cu) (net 6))
 (segment (start 68.58 71.12) (end 59.69 62.23) (width 0.254) (layer B.Cu) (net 7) (status 10))
 (segment (start 63.5 45.72) (end 63.5 43.66) (width 0.254) (layer B.Cu) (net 7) (status 20))
 (segment (start 59.69 49.53) (end 63.5 45.72) (width 0.254) (layer B.Cu) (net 7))
 (segment (start 59.69 62.23) (end 59.69 49.53) (width 0.254) (layer B.Cu) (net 7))
 (segment (start 60.96 50.8) (end 66.04 45.72) (width 0.254) (layer B.Cu) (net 8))
 (segment (start 66.04 45.72) (end 66.04 43.66) (width 0.254) (layer B.Cu) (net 8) (status 20))
 (segment (start 68.58 68.58) (end 60.96 60.96) (width 0.254) (layer B.Cu) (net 8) (status 10))
 (segment (start 60.96 60.96) (end 60.96 50.8) (width 0.254) (layer B.Cu) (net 8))
 (segment (start 76.2 66.04) (end 77.47 66.04) (width 0.254) (layer B.Cu) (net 19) (status 10))
 (segment (start 77.47 66.04) (end 85.09 58.42) (width 0.254) (layer B.Cu) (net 19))
 (via (at 85.09 48.26) (size 0.889) (layers F.Cu B.Cu) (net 19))
 (segment (start 85.09 58.42) (end 85.09 48.26) (width 0.254) (layer B.Cu) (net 19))
 (segment (start 85.09 48.26) (end 91.44 48.26) (width 0.254) (layer F.Cu) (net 19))
 (segment (start 93.98 45.72) (end 95.25 45.72) (width 0.254) (layer F.Cu) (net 19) (status 20))
 (segment (start 91.44 48.26) (end 93.98 45.72) (width 0.254) (layer F.Cu) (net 19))
 (segment (start 53.34 48.26) (end 50.8 45.72) (width 0.254) (layer F.Cu) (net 19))
 (segment (start 50.8 45.72) (end 49.53 45.72) (width 0.254) (layer F.Cu) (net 19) (status 20))
 (segment (start 53.34 48.26) (end 85.09 48.26) (width 0.254) (layer F.Cu) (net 19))
 (segment (start 76.2 63.5) (end 77.47 63.5) (width 0.254) (layer B.Cu) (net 18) (status 10))
 (segment (start 83.82 57.15) (end 77.47 63.5) (width 0.254) (layer B.Cu) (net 18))
 (segment (start 93.98 43.18) (end 95.25 43.18) (width 0.254) (layer F.Cu) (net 18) (status 20))
 (segment (start 54.61 46.99) (end 50.8 43.18) (width 0.254) (layer F.Cu) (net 18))
 (segment (start 50.8 43.18) (end 49.53 43.18) (width 0.254) (layer F.Cu) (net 18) (status 20))
 (via (at 83.82 46.99) (size 0.889) (layers F.Cu B.Cu) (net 18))
 (segment (start 83.82 57.15) (end 83.82 46.99) (width 0.254) (layer B.Cu) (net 18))
 (segment (start 54.61 46.99) (end 83.82 46.99) (width 0.254) (layer F.Cu) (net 18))
 (segment (start 90.17 46.99) (end 93.98 43.18) (width 0.254) (layer F.Cu) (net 18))
 (segment (start 83.82 46.99) (end 90.17 46.99) (width 0.254) (layer F.Cu) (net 18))
 (segment (start 76.2 81.28) (end 77.47 81.28) (width 0.254) (layer B.Cu) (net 25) (status 10))
 (segment (start 81.28 85.09) (end 77.47 81.28) (width 0.254) (layer B.Cu) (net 25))
 (via (at 81.28 93.98) (size 0.889) (layers F.Cu B.Cu) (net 25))
 (segment (start 81.28 85.09) (end 81.28 93.98) (width 0.254) (layer B.Cu) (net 25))
 (segment (start 67.31 93.98) (end 81.28 93.98) (width 0.254) (layer F.Cu) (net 25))
 (segment (start 66.04 92.71) (end 67.31 93.98) (width 0.254) (layer F.Cu) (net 25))
 (segment (start 66.04 54.61) (end 66.04 92.71) (width 0.254) (layer F.Cu) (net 25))
 (segment (start 81.28 93.98) (end 88.9 93.98) (width 0.254) (layer F.Cu) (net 25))
 (segment (start 90.17 58.42) (end 95.25 53.34) (width 0.254) (layer F.Cu) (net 25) (status 20))
 (segment (start 90.17 92.71) (end 90.17 58.42) (width 0.254) (layer F.Cu) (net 25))
 (segment (start 88.9 93.98) (end 90.17 92.71) (width 0.254) (layer F.Cu) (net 25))
 (segment (start 49.53 53.34) (end 64.77 53.34) (width 0.254) (layer F.Cu) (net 25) (status 10))
 (segment (start 64.77 53.34) (end 66.04 54.61) (width 0.254) (layer F.Cu) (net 25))
 (segment (start 49.53 55.88) (end 63.5 55.88) (width 0.254) (layer F.Cu) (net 26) (status 10))
 (segment (start 63.5 55.88) (end 64.77 57.15) (width 0.254) (layer F.Cu) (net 26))
 (segment (start 64.77 57.15) (end 64.77 92.71) (width 0.254) (layer F.Cu) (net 26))
 (via (at 80.01 95.25) (size 0.889) (layers F.Cu B.Cu) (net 26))
 (segment (start 76.2 83.82) (end 77.47 83.82) (width 0.254) (layer B.Cu) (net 26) (status 10))
 (segment (start 80.01 86.36) (end 77.47 83.82) (width 0.254) (layer B.Cu) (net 26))
 (segment (start 80.01 86.36) (end 80.01 95.25) (width 0.254) (layer B.Cu) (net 26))
 (segment (start 67.31 95.25) (end 80.01 95.25) (width 0.254) (layer F.Cu) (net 26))
 (segment (start 64.77 92.71) (end 67.31 95.25) (width 0.254) (layer F.Cu) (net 26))
 (segment (start 90.17 55.88) (end 95.25 55.88) (width 0.254) (layer B.Cu) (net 17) (status 20))
 (via (at 90.17 55.88) (size 0.889) (layers F.Cu B.Cu) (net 17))
 (segment (start 76.2 60.96) (end 77.47 60.96) (width 0.254) (layer F.Cu) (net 17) (status 10))
 (segment (start 77.47 60.96) (end 82.55 55.88) (width 0.254) (layer F.Cu) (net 17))
 (segment (start 82.55 55.88) (end 90.17 55.88) (width 0.254) (layer F.Cu) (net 17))
 (segment (start 49.53 58.42) (end 62.23 58.42) (width 0.254) (layer F.Cu) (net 27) (status 10))
 (segment (start 78.74 96.52) (end 90.17 96.52) (width 0.254) (layer F.Cu) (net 27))
 (segment (start 91.44 62.23) (end 95.25 58.42) (width 0.254) (layer F.Cu) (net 27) (status 20))
 (segment (start 91.44 95.25) (end 91.44 62.23) (width 0.254) (layer F.Cu) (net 27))
 (segment (start 90.17 96.52) (end 91.44 95.25) (width 0.254) (layer F.Cu) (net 27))
 (via (at 78.74 96.52) (size 0.889) (layers F.Cu B.Cu) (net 27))
 (segment (start 78.74 87.63) (end 78.74 96.52) (width 0.254) (layer B.Cu) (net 27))
 (segment (start 66.04 96.52) (end 78.74 96.52) (width 0.254) (layer F.Cu) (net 27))
 (segment (start 63.5 93.98) (end 66.04 96.52) (width 0.254) (layer F.Cu) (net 27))
 (segment (start 78.74 87.63) (end 77.47 86.36) (width 0.254) (layer B.Cu) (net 27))
 (segment (start 63.5 59.69) (end 63.5 93.98) (width 0.254) (layer F.Cu) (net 27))
 (segment (start 62.23 58.42) (end 63.5 59.69) (width 0.254) (layer F.Cu) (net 27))
 (segment (start 76.2 86.36) (end 77.47 86.36) (width 0.254) (layer B.Cu) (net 27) (status 10))
 (segment (start 76.2 58.42) (end 77.47 58.42) (width 0.254) (layer B.Cu) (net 16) (status 10))
 (segment (start 82.55 53.34) (end 77.47 58.42) (width 0.254) (layer B.Cu) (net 16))
 (segment (start 93.98 40.64) (end 95.25 40.64) (width 0.254) (layer F.Cu) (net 16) (status 20))
 (segment (start 55.88 45.72) (end 50.8 40.64) (width 0.254) (layer F.Cu) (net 16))
 (segment (start 50.8 40.64) (end 49.53 40.64) (width 0.254) (layer F.Cu) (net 16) (status 20))
 (via (at 82.55 45.72) (size 0.889) (layers F.Cu B.Cu) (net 16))
 (segment (start 82.55 53.34) (end 82.55 45.72) (width 0.254) (layer B.Cu) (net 16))
 (segment (start 55.88 45.72) (end 82.55 45.72) (width 0.254) (layer F.Cu) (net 16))
 (segment (start 88.9 45.72) (end 93.98 40.64) (width 0.254) (layer F.Cu) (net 16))
 (segment (start 82.55 45.72) (end 88.9 45.72) (width 0.254) (layer F.Cu) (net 16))
 (segment (start 49.53 50.8) (end 87.63 50.8) (width 0.254) (layer F.Cu) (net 24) (status 10))
 (segment (start 87.63 50.8) (end 95.25 50.8) (width 0.254) (layer F.Cu) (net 24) (status 20))
 (via (at 87.63 50.8) (size 0.889) (layers F.Cu B.Cu) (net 24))
 (segment (start 87.63 59.69) (end 87.63 50.8) (width 0.254) (layer B.Cu) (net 24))
 (segment (start 76.2 78.74) (end 86.36 78.74) (width 0.254) (layer F.Cu) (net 24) (status 10))
 (segment (start 87.63 77.47) (end 87.63 59.69) (width 0.254) (layer F.Cu) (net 24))
 (segment (start 86.36 78.74) (end 87.63 77.47) (width 0.254) (layer F.Cu) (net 24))
 (via (at 87.63 59.69) (size 0.889) (layers F.Cu B.Cu) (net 24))
 (segment (start 52.07 96.52) (end 53.34 97.79) (width 0.254) (layer F.Cu) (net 22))
 (segment (start 50.8 60.96) (end 52.07 62.23) (width 0.254) (layer F.Cu) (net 22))
 (segment (start 52.07 62.23) (end 52.07 96.52) (width 0.254) (layer F.Cu) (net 22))
 (segment (start 49.53 60.96) (end 50.8 60.96) (width 0.254) (layer F.Cu) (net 22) (status 10))
 (segment (start 92.71 63.5) (end 95.25 60.96) (width 0.254) (layer F.Cu) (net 22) (status 20))
 (segment (start 92.71 72.39) (end 92.71 63.5) (width 0.254) (layer F.Cu) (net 22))
 (via (at 88.9 73.66) (size 0.889) (layers F.Cu B.Cu) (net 22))
 (segment (start 87.63 85.09) (end 88.9 83.82) (width 0.254) (layer F.Cu) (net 22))
 (segment (start 88.9 83.82) (end 88.9 73.66) (width 0.254) (layer F.Cu) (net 22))
 (segment (start 80.01 73.66) (end 88.9 73.66) (width 0.254) (layer B.Cu) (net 22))
 (segment (start 88.9 73.66) (end 92.71 73.66) (width 0.254) (layer B.Cu) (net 22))
 (via (at 92.71 73.66) (size 0.889) (layers F.Cu B.Cu) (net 22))
 (segment (start 76.2 73.66) (end 80.01 73.66) (width 0.254) (layer B.Cu) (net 22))
 (segment (start 92.71 96.52) (end 92.71 73.66) (width 0.254) (layer F.Cu) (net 22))
 (segment (start 91.44 97.79) (end 92.71 96.52) (width 0.254) (layer F.Cu) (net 22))
 (segment (start 53.34 97.79) (end 91.44 97.79) (width 0.254) (layer F.Cu) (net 22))
 (segment (start 92.71 73.66) (end 92.71 72.39) (width 0.254) (layer F.Cu) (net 22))
 (segment (start 80.01 71.12) (end 82.55 71.12) (width 0.254) (layer F.Cu) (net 20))
 (segment (start 83.82 83.82) (end 85.09 85.09) (width 0.254) (layer B.Cu) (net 20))
 (segment (start 83.82 74.93) (end 83.82 83.82) (width 0.254) (layer B.Cu) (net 20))
 (via (at 83.82 74.93) (size 0.889) (layers F.Cu B.Cu) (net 20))
 (segment (start 83.82 72.39) (end 83.82 74.93) (width 0.254) (layer F.Cu) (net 20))
 (segment (start 82.55 71.12) (end 83.82 72.39) (width 0.254) (layer F.Cu) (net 20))
 (segment (start 76.2 68.58) (end 77.47 68.58) (width 0.254) (layer F.Cu) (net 20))
 (segment (start 77.47 68.58) (end 80.01 71.12) (width 0.254) (layer F.Cu) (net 20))
 (segment (start 49.53 63.5) (end 49.53 97.79) (width 0.254) (layer F.Cu) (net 21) (status 10))
 (segment (start 49.53 63.5) (end 55.88 63.5) (width 0.254) (layer B.Cu) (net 21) (status 10))
 (segment (start 55.88 63.5) (end 57.15 62.23) (width 0.254) (layer B.Cu) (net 21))
 (segment (start 57.15 62.23) (end 57.15 43.18) (width 0.254) (layer B.Cu) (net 21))
 (segment (start 82.55 63.5) (end 85.09 63.5) (width 0.254) (layer B.Cu) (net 21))
 (segment (start 78.74 67.31) (end 82.55 63.5) (width 0.254) (layer B.Cu) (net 21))
 (segment (start 85.09 63.5) (end 95.25 63.5) (width 0.254) (layer B.Cu) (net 21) (status 20))
 (segment (start 95.25 63.5) (end 95.25 97.79) (width 0.254) (layer F.Cu) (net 21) (status 10))
 (segment (start 93.98 99.06) (end 60.96 99.06) (width 0.254) (layer F.Cu) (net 21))
 (segment (start 93.98 99.06) (end 95.25 97.79) (width 0.254) (layer F.Cu) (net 21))
 (segment (start 50.8 99.06) (end 60.96 99.06) (width 0.254) (layer F.Cu) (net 21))
 (segment (start 76.2 71.12) (end 78.74 68.58) (width 0.254) (layer B.Cu) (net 21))
 (segment (start 78.74 68.58) (end 78.74 67.31) (width 0.254) (layer B.Cu) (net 21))
 (segment (start 49.53 97.79) (end 50.8 99.06) (width 0.254) (layer F.Cu) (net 21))
 (segment (start 60.96 99.06) (end 60.96 103.66) (width 0.254) (layer F.Cu) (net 21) (status 20))
 (segment (start 82.07 41.91) (end 83.82 43.66) (width 0.254) (layer B.Cu) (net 21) (status 20))
 (segment (start 58.42 41.91) (end 82.07 41.91) (width 0.254) (layer B.Cu) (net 21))
 (segment (start 57.15 43.18) (end 58.42 41.91) (width 0.254) (layer B.Cu) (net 21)))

